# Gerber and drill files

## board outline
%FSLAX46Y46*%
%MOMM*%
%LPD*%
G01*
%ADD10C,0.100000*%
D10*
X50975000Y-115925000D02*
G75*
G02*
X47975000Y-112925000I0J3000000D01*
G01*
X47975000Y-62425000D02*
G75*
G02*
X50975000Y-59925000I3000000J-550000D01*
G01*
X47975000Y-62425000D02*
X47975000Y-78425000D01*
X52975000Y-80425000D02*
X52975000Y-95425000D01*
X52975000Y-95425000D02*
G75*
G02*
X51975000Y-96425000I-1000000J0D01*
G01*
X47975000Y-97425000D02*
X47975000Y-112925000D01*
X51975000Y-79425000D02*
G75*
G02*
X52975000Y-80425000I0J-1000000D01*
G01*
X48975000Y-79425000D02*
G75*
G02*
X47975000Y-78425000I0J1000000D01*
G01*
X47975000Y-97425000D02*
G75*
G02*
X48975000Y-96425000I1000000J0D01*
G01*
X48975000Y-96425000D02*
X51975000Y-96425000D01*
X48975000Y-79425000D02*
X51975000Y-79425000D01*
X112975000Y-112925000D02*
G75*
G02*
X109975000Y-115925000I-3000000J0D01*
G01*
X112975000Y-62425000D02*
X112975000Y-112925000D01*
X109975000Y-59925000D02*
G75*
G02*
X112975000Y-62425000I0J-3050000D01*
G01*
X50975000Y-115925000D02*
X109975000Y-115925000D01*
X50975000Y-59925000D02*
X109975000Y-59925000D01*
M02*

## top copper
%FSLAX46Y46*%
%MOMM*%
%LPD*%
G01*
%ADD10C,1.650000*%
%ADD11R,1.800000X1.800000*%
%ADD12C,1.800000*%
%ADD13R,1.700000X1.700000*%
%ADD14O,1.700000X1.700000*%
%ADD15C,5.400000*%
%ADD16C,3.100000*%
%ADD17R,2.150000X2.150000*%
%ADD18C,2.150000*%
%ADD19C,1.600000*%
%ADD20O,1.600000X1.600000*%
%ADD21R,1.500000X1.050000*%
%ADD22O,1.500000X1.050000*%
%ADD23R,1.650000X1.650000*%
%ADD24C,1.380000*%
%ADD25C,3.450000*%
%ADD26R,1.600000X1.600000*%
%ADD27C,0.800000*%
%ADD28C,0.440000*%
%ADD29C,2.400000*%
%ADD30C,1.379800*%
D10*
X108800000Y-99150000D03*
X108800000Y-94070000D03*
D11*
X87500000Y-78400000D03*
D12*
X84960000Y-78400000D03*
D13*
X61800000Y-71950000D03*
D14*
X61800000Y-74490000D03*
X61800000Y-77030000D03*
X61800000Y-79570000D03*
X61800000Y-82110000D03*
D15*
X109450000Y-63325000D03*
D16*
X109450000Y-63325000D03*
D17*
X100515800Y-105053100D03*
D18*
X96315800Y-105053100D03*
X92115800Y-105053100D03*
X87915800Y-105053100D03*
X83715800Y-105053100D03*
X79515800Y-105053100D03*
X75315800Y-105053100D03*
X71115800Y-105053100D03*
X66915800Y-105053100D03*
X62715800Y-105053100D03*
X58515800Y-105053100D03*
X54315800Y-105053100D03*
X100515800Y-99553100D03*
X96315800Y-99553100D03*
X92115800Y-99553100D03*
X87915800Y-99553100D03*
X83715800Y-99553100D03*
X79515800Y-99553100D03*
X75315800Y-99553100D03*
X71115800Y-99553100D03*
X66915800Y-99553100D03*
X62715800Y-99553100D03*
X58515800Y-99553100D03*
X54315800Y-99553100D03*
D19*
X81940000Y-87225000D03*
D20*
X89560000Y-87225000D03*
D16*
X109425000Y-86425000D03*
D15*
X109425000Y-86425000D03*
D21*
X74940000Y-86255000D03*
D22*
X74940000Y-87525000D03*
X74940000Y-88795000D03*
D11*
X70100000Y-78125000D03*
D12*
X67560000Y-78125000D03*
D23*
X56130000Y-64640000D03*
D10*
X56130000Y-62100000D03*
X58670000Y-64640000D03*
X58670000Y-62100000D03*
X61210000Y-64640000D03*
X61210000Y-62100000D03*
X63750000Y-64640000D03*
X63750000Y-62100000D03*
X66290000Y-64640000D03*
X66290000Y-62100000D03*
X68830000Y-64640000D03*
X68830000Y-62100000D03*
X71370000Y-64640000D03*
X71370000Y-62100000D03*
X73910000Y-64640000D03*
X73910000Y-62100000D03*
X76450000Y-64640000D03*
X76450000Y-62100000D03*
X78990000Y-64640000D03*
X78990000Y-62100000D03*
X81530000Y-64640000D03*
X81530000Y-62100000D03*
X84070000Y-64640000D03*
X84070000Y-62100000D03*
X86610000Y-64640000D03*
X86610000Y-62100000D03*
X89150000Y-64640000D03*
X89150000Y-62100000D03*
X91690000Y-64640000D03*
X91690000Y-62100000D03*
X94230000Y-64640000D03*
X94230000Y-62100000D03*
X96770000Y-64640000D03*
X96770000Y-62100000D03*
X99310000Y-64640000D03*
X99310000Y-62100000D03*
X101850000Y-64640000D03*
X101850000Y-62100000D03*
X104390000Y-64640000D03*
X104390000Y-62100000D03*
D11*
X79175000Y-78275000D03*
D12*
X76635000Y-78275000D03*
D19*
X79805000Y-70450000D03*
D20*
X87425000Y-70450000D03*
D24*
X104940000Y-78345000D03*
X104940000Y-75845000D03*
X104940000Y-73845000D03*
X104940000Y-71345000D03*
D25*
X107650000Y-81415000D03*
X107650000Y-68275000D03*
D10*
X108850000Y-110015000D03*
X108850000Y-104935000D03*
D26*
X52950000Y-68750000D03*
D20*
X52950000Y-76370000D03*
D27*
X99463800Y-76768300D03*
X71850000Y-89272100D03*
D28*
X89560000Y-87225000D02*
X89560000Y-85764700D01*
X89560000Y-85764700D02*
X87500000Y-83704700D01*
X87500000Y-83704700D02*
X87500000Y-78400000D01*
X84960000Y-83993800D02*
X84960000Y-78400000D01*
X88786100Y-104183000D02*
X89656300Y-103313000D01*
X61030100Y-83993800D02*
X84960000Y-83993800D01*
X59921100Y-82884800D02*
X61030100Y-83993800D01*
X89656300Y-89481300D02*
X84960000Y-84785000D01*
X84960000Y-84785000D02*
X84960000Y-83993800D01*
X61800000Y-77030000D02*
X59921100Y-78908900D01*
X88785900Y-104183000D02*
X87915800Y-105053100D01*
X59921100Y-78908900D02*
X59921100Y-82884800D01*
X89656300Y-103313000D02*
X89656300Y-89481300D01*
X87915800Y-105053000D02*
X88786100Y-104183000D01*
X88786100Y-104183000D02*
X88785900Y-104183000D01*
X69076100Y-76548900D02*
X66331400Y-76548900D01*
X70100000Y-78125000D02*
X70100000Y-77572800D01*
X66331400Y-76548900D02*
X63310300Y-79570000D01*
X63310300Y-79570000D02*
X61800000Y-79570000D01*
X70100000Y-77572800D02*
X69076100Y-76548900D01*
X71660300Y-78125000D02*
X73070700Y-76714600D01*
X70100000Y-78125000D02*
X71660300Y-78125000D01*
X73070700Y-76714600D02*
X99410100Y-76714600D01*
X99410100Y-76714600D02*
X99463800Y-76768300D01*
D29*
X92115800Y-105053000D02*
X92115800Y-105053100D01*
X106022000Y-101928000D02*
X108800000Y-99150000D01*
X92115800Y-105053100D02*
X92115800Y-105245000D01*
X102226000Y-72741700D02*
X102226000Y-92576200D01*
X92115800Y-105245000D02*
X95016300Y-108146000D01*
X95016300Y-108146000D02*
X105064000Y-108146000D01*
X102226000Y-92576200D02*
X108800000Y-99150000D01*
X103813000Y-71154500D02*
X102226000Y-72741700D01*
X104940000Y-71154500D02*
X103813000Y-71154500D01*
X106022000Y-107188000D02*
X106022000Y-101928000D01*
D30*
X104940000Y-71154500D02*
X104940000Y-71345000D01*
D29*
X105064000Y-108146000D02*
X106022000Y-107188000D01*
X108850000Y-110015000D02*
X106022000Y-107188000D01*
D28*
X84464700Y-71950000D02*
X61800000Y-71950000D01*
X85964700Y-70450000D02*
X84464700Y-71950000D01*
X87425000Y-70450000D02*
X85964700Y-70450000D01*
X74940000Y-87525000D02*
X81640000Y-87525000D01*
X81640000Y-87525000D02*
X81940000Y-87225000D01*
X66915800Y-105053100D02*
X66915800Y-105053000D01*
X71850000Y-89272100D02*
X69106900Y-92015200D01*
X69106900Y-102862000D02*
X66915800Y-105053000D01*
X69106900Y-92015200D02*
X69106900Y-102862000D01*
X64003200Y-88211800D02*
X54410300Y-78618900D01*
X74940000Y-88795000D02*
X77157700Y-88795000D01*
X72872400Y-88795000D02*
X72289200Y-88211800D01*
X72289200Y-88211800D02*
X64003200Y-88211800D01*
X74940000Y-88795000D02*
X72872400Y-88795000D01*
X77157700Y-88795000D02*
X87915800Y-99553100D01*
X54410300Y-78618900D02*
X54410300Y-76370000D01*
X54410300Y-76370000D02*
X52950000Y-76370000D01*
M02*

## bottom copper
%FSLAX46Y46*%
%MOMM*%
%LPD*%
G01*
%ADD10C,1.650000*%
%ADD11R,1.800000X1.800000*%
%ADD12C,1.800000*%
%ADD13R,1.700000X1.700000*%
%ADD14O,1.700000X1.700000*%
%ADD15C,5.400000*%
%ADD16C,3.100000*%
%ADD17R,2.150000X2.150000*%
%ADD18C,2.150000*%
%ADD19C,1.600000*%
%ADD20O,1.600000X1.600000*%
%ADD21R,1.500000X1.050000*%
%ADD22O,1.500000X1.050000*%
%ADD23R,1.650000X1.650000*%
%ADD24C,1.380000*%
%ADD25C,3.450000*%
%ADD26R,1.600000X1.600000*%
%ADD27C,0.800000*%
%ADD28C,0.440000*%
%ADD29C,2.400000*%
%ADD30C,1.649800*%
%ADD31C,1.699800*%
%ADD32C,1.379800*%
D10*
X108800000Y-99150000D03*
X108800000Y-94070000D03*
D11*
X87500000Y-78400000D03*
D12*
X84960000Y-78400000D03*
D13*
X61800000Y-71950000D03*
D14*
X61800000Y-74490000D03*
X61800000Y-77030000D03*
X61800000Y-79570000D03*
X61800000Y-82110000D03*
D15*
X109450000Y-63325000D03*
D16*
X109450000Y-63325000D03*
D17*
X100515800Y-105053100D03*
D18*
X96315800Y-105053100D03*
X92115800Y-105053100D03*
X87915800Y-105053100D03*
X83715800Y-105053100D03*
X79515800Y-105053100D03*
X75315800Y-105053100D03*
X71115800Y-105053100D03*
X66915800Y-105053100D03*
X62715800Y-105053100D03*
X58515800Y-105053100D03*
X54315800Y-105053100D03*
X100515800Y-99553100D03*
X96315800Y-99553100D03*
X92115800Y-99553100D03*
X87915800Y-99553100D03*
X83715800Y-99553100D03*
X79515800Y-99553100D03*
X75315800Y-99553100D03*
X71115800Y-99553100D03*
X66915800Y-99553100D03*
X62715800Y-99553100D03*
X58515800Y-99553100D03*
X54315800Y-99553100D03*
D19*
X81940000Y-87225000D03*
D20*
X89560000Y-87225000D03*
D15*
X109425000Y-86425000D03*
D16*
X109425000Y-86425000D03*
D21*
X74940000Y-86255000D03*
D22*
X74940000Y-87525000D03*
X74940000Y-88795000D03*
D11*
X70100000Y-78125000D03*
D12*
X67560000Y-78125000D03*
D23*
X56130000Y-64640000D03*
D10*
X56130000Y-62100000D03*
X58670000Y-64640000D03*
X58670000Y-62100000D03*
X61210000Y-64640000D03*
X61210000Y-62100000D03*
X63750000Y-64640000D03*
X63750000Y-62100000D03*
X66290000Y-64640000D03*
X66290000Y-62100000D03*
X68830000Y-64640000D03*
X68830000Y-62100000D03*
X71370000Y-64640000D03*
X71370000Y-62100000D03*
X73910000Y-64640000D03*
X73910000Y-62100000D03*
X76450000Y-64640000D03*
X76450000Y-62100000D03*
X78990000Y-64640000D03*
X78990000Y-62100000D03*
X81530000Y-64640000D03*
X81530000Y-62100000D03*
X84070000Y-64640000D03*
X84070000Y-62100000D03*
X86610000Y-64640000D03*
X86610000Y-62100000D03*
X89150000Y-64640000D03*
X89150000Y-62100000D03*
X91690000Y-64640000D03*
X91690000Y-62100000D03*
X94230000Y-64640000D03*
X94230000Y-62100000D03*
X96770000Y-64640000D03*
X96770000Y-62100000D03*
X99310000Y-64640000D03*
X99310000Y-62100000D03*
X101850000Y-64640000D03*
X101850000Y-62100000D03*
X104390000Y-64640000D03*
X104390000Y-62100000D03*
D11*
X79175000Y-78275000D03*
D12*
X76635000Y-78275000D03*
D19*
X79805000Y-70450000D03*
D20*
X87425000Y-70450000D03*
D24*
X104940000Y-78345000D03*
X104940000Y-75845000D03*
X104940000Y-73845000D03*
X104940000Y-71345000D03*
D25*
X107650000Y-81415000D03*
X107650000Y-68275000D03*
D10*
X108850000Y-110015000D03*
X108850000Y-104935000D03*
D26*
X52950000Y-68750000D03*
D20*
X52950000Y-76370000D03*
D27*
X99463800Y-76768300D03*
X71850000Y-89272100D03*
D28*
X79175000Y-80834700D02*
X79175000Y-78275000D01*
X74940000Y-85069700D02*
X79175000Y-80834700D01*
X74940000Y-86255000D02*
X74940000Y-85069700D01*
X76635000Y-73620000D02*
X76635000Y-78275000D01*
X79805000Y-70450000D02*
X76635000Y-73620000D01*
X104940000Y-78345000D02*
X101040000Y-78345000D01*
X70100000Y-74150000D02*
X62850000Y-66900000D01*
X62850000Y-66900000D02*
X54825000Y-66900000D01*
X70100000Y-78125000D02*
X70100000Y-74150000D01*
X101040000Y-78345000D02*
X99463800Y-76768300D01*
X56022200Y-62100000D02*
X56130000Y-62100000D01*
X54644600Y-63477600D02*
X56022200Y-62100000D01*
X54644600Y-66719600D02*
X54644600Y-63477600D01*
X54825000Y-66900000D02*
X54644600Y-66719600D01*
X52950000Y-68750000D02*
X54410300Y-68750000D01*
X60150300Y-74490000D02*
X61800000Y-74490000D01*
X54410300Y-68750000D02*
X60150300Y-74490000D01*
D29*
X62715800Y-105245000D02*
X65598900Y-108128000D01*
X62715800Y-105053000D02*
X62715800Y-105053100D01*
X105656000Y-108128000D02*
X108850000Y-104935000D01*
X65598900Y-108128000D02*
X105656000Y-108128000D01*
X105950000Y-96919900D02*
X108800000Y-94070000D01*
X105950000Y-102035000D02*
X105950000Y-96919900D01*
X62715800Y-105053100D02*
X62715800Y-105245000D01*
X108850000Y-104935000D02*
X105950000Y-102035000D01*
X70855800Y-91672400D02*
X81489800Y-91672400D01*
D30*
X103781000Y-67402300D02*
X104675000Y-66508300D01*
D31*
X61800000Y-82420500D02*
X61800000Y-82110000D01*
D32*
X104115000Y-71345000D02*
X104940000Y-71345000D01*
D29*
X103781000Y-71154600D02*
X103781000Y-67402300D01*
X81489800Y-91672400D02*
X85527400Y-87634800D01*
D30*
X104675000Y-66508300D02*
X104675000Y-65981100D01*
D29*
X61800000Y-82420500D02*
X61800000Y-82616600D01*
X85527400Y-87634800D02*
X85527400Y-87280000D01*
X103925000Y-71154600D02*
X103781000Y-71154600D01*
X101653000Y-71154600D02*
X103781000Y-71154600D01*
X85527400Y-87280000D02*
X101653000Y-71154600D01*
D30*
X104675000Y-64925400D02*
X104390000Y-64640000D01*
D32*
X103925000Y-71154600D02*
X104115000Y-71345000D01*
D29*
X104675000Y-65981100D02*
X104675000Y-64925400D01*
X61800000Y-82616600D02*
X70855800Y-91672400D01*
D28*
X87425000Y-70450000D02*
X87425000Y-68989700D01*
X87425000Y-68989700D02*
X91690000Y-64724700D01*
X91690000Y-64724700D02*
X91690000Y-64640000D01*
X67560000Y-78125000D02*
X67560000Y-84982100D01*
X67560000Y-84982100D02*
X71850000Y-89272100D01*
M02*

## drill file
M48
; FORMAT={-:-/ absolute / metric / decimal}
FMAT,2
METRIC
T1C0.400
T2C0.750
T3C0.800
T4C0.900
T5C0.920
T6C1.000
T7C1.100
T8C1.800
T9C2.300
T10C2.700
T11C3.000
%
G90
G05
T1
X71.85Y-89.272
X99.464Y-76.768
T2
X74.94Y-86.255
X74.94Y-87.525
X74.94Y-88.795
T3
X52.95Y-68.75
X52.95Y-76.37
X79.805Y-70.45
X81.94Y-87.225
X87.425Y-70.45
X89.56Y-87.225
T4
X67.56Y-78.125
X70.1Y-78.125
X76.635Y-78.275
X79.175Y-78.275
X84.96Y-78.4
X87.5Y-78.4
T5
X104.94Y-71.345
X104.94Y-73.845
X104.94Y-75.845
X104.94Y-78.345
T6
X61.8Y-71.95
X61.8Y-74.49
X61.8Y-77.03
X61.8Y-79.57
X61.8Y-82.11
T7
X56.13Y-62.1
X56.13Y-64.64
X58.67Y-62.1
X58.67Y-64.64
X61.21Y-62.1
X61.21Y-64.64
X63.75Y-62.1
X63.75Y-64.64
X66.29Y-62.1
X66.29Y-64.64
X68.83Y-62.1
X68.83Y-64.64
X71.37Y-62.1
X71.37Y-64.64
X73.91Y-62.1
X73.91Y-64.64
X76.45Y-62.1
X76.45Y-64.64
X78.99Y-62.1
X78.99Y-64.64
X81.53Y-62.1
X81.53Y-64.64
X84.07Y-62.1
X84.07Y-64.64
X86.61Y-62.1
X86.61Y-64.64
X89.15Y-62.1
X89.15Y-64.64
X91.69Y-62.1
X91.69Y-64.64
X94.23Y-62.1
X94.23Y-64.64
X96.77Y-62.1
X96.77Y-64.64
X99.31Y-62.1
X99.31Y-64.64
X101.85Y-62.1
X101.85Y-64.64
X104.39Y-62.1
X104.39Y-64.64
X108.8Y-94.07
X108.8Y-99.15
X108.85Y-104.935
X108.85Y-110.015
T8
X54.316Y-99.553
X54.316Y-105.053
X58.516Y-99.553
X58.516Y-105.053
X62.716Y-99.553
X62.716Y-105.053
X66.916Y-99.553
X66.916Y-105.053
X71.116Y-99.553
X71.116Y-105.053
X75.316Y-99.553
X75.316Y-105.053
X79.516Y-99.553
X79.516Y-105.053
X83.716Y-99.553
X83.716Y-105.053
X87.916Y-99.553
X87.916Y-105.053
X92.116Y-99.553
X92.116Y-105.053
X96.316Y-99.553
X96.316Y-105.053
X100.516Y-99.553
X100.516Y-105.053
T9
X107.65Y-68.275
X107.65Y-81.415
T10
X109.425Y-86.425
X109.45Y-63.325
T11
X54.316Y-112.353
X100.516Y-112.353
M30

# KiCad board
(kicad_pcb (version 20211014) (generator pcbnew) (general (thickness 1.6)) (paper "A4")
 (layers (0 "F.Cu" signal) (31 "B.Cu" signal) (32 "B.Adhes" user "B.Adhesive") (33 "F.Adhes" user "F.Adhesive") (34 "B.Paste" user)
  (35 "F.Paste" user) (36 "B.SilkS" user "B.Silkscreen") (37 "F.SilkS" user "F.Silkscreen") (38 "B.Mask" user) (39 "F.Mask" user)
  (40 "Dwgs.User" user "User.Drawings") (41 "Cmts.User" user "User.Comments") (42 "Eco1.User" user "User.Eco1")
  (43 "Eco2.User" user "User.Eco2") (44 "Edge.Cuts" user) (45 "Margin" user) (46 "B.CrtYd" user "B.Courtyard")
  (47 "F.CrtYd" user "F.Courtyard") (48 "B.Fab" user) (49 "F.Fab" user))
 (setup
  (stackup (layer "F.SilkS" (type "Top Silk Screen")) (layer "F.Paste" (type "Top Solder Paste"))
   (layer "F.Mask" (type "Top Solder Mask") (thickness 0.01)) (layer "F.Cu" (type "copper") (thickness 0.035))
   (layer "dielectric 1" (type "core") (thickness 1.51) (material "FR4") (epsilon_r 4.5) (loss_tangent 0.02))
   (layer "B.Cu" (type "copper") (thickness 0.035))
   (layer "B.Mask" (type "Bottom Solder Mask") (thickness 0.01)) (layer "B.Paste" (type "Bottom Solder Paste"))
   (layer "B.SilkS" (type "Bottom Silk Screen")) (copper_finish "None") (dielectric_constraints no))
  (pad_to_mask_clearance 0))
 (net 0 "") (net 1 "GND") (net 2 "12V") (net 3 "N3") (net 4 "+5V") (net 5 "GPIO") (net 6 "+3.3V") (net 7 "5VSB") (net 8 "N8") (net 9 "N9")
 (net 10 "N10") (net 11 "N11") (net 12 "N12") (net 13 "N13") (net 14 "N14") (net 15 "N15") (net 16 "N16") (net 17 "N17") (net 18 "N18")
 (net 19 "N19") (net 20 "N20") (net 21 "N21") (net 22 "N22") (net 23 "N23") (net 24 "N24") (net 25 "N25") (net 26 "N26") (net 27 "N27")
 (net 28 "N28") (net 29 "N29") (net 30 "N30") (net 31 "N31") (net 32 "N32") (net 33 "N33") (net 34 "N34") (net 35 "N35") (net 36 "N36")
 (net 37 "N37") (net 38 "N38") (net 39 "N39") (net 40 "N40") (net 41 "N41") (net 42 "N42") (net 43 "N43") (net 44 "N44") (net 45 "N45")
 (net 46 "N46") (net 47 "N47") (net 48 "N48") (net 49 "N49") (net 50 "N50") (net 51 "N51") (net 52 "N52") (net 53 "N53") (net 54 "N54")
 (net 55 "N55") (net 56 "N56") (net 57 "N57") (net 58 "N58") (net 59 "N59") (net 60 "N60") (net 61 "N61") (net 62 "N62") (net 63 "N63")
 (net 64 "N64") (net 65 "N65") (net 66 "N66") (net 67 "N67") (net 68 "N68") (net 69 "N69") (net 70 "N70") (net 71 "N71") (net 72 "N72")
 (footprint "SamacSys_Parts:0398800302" (layer "F.Cu") (at 108.8 99.15 90)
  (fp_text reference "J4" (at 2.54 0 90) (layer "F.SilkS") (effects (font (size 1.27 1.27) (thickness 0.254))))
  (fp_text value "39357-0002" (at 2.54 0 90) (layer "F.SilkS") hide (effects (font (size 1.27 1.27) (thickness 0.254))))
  (pad "1" thru_hole circle locked (at 0 0 90) (size 1.65 1.65) (drill 1.1) (layers *.Cu *.Mask) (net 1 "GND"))
  (pad "2" thru_hole circle locked (at 5.08 0 90) (size 1.65 1.65) (drill 1.1) (layers *.Cu *.Mask) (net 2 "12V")))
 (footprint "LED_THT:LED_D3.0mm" (layer "F.Cu") (at 87.5 78.4 180)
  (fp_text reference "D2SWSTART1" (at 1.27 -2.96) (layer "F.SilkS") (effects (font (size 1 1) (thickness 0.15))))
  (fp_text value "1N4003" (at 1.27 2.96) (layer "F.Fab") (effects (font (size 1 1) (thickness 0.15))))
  (pad "1" thru_hole rect (at 0 0 180) (size 1.8 1.8) (drill 0.9) (layers *.Cu *.Mask) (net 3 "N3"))
  (pad "2" thru_hole circle (at 2.54 0 180) (size 1.8 1.8) (drill 0.9) (layers *.Cu *.Mask) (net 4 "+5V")))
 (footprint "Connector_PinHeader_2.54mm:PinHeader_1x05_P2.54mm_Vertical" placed (layer "F.Cu") (at 61.8 71.95)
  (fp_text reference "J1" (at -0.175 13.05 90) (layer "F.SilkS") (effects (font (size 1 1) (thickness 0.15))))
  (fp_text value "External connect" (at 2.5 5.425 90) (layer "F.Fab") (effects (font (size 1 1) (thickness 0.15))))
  (pad "1" thru_hole rect (at 0 0) (size 1.7 1.7) (drill 1) (layers *.Cu *.Mask) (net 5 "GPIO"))
  (pad "2" thru_hole oval (at 0 2.54) (size 1.7 1.7) (drill 1) (layers *.Cu *.Mask) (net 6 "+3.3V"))
  (pad "3" thru_hole oval (at 0 5.08) (size 1.7 1.7) (drill 1) (layers *.Cu *.Mask) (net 4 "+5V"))
  (pad "4" thru_hole oval (at 0 7.62) (size 1.7 1.7) (drill 1) (layers *.Cu *.Mask) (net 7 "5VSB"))
  (pad "5" thru_hole oval (at 0 10.16) (size 1.7 1.7) (drill 1) (layers *.Cu *.Mask) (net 1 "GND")))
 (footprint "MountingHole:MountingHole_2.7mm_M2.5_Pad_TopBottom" (layer "F.Cu") (at 109.45 63.325)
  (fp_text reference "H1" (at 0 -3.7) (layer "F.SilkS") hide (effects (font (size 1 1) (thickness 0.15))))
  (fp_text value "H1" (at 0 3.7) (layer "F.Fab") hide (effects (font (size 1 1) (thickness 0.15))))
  (pad "1" connect circle (at 0 0) (size 5.4 5.4) (layers "B.Cu" "B.Mask"))
  (pad "1" connect circle (at 0 0) (size 5.4 5.4) (layers "F.Cu" "F.Mask"))
  (pad "1" thru_hole circle (at 0 0) (size 3.1 3.1) (drill 2.7) (layers *.Cu *.Mask)))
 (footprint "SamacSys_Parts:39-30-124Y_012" (layer "F.Cu") (at 100.5158 105.0531)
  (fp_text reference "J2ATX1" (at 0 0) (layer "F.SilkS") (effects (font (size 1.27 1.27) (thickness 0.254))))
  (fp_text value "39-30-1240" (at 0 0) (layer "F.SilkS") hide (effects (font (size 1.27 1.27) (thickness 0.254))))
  (pad "" np_thru_hole circle locked (at 0 7.3) (size 3 3) (drill 3) (layers *.Cu *.Mask))
  (pad "" np_thru_hole circle locked (at -46.2 7.3) (size 3 3) (drill 3) (layers *.Cu *.Mask))
  (pad "1" thru_hole rect locked (at 0 0) (size 2.15 2.15) (drill 1.8) (layers *.Cu *.Mask) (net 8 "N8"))
  (pad "2" thru_hole circle locked (at -4.2 0) (size 2.15 2.15) (drill 1.8) (layers *.Cu *.Mask) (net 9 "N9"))
  (pad "3" thru_hole circle locked (at -8.4 0) (size 2.15 2.15) (drill 1.8) (layers *.Cu *.Mask) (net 1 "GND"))
  (pad "4" thru_hole circle locked (at -12.6 0) (size 2.15 2.15) (drill 1.8) (layers *.Cu *.Mask) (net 4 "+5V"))
  (pad "5" thru_hole circle locked (at -16.8 0) (size 2.15 2.15) (drill 1.8) (layers *.Cu *.Mask) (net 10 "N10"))
  (pad "6" thru_hole circle locked (at -21 0) (size 2.15 2.15) (drill 1.8) (layers *.Cu *.Mask) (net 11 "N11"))
  (pad "7" thru_hole circle locked (at -25.2 0) (size 2.15 2.15) (drill 1.8) (layers *.Cu *.Mask) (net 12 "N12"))
  (pad "8" thru_hole circle locked (at -29.4 0) (size 2.15 2.15) (drill 1.8) (layers *.Cu *.Mask) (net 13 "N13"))
  (pad "9" thru_hole circle locked (at -33.6 0) (size 2.15 2.15) (drill 1.8) (layers *.Cu *.Mask) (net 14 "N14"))
  (pad "10" thru_hole circle locked (at -37.8 0) (size 2.15 2.15) (drill 1.8) (layers *.Cu *.Mask) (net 2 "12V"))
  (pad "11" thru_hole circle locked (at -42 0) (size 2.15 2.15) (drill 1.8) (layers *.Cu *.Mask) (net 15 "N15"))
  (pad "12" thru_hole circle locked (at -46.2 0) (size 2.15 2.15) (drill 1.8) (layers *.Cu *.Mask) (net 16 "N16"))
  (pad "13" thru_hole circle locked (at 0 -5.5) (size 2.15 2.15) (drill 1.8) (layers *.Cu *.Mask) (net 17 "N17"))
  (pad "14" thru_hole circle locked (at -4.2 -5.5) (size 2.15 2.15) (drill 1.8) (layers *.Cu *.Mask) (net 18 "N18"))
  (pad "15" thru_hole circle locked (at -8.4 -5.5) (size 2.15 2.15) (drill 1.8) (layers *.Cu *.Mask) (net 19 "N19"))
  (pad "16" thru_hole circle locked (at -12.6 -5.5) (size 2.15 2.15) (drill 1.8) (layers *.Cu *.Mask) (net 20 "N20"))
  (pad "17" thru_hole circle locked (at -16.8 -5.5) (size 2.15 2.15) (drill 1.8) (layers *.Cu *.Mask) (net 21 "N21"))
  (pad "18" thru_hole circle locked (at -21 -5.5) (size 2.15 2.15) (drill 1.8) (layers *.Cu *.Mask) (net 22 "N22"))
  (pad "19" thru_hole circle locked (at -25.2 -5.5) (size 2.15 2.15) (drill 1.8) (layers *.Cu *.Mask) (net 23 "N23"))
  (pad "20" thru_hole circle locked (at -29.4 -5.5) (size 2.15 2.15) (drill 1.8) (layers *.Cu *.Mask) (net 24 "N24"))
  (pad "21" thru_hole circle locked (at -33.6 -5.5) (size 2.15 2.15) (drill 1.8) (layers *.Cu *.Mask) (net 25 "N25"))
  (pad "22" thru_hole circle locked (at -37.8 -5.5) (size 2.15 2.15) (drill 1.8) (layers *.Cu *.Mask) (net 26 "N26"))
  (pad "23" thru_hole circle locked (at -42 -5.5) (size 2.15 2.15) (drill 1.8) (layers *.Cu *.Mask) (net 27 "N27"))
  (pad "24" thru_hole circle locked (at -46.2 -5.5) (size 2.15 2.15) (drill 1.8) (layers *.Cu *.Mask) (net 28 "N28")))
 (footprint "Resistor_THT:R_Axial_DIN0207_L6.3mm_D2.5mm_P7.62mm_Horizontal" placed (layer "F.Cu") (at 81.94 87.225)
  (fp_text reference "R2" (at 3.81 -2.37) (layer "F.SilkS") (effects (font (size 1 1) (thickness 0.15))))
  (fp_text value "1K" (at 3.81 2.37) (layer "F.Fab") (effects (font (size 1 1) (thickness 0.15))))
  (pad "1" thru_hole circle (at 0 0) (size 1.6 1.6) (drill 0.8) (layers *.Cu *.Mask) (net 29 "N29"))
  (pad "2" thru_hole oval (at 7.62 0) (size 1.6 1.6) (drill 0.8) (layers *.Cu *.Mask) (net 3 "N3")))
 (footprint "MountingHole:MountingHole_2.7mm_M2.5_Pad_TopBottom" (layer "F.Cu") (at 109.425 86.425)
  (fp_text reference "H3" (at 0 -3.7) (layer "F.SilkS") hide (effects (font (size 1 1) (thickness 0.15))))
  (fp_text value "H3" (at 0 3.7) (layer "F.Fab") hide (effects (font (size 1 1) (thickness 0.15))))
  (pad "1" connect circle (at 0 0) (size 5.4 5.4) (layers "B.Cu" "B.Mask"))
  (pad "3" thru_hole circle (at 0 0) (size 3.1 3.1) (drill 2.7) (layers *.Cu *.Mask))
  (pad "3" connect circle (at 0 0) (size 5.4 5.4) (layers "F.Cu" "F.Mask")))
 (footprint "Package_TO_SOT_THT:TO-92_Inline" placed (layer "F.Cu") (at 74.94 86.255 -90)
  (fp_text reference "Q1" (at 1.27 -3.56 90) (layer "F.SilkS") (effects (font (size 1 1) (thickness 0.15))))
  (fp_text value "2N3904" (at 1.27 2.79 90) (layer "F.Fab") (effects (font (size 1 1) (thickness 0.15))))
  (pad "1" thru_hole rect (at 0 0 270) (size 1.05 1.5) (drill 0.75) (layers *.Cu *.Mask) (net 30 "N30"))
  (pad "2" thru_hole oval (at 1.27 0 270) (size 1.05 1.5) (drill 0.75) (layers *.Cu *.Mask) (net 29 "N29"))
  (pad "3" thru_hole oval (at 2.54 0 270) (size 1.05 1.5) (drill 0.75) (layers *.Cu *.Mask) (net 20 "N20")))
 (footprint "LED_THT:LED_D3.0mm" (layer "F.Cu") (at 70.1 78.125 180)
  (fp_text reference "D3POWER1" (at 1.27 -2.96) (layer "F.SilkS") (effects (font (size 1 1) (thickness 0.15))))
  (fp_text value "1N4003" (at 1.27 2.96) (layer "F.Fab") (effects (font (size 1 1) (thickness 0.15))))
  (pad "1" thru_hole rect (at 0 0 180) (size 1.8 1.8) (drill 0.9) (layers *.Cu *.Mask) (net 7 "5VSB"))
  (pad "2" thru_hole circle (at 2.54 0 180) (size 1.8 1.8) (drill 0.9) (layers *.Cu *.Mask) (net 14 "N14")))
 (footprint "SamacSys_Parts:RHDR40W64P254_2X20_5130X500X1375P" (layer "F.Cu") (at 56.13 64.64)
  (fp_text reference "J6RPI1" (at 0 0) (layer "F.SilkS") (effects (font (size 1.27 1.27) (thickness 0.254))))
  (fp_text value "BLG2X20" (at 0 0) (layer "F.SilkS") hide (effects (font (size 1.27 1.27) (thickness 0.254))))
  (pad "1" thru_hole rect locked (at 0 0) (size 1.65 1.65) (drill 1.1) (layers *.Cu *.Mask) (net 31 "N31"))
  (pad "2" thru_hole circle locked (at 0 -2.54) (size 1.65 1.65) (drill 1.1) (layers *.Cu *.Mask) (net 7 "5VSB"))
  (pad "3" thru_hole circle locked (at 2.54 0) (size 1.65 1.65) (drill 1.1) (layers *.Cu *.Mask) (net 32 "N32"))
  (pad "4" thru_hole circle locked (at 2.54 -2.54) (size 1.65 1.65) (drill 1.1) (layers *.Cu *.Mask) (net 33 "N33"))
  (pad "5" thru_hole circle locked (at 5.08 0) (size 1.65 1.65) (drill 1.1) (layers *.Cu *.Mask) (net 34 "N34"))
  (pad "6" thru_hole circle locked (at 5.08 -2.54) (size 1.65 1.65) (drill 1.1) (layers *.Cu *.Mask) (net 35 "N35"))
  (pad "7" thru_hole circle locked (at 7.62 0) (size 1.65 1.65) (drill 1.1) (layers *.Cu *.Mask) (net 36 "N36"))
  (pad "8" thru_hole circle locked (at 7.62 -2.54) (size 1.65 1.65) (drill 1.1) (layers *.Cu *.Mask) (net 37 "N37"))
  (pad "9" thru_hole circle locked (at 10.16 0) (size 1.65 1.65) (drill 1.1) (layers *.Cu *.Mask) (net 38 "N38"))
  (pad "10" thru_hole circle locked (at 10.16 -2.54) (size 1.65 1.65) (drill 1.1) (layers *.Cu *.Mask) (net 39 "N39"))
  (pad "11" thru_hole circle locked (at 12.7 0) (size 1.65 1.65) (drill 1.1) (layers *.Cu *.Mask) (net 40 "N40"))
  (pad "12" thru_hole circle locked (at 12.7 -2.54) (size 1.65 1.65) (drill 1.1) (layers *.Cu *.Mask) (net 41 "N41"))
  (pad "13" thru_hole circle locked (at 15.24 0) (size 1.65 1.65) (drill 1.1) (layers *.Cu *.Mask) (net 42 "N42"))
  (pad "14" thru_hole circle locked (at 15.24 -2.54) (size 1.65 1.65) (drill 1.1) (layers *.Cu *.Mask) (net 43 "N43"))
  (pad "15" thru_hole circle locked (at 17.78 0) (size 1.65 1.65) (drill 1.1) (layers *.Cu *.Mask) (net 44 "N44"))
  (pad "16" thru_hole circle locked (at 17.78 -2.54) (size 1.65 1.65) (drill 1.1) (layers *.Cu *.Mask) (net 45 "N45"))
  (pad "17" thru_hole circle locked (at 20.32 0) (size 1.65 1.65) (drill 1.1) (layers *.Cu *.Mask) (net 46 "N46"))
  (pad "18" thru_hole circle locked (at 20.32 -2.54) (size 1.65 1.65) (drill 1.1) (layers *.Cu *.Mask) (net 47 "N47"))
  (pad "19" thru_hole circle locked (at 22.86 0) (size 1.65 1.65) (drill 1.1) (layers *.Cu *.Mask) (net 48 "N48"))
  (pad "20" thru_hole circle locked (at 22.86 -2.54) (size 1.65 1.65) (drill 1.1) (layers *.Cu *.Mask) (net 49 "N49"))
  (pad "21" thru_hole circle locked (at 25.4 0) (size 1.65 1.65) (drill 1.1) (layers *.Cu *.Mask) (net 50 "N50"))
  (pad "22" thru_hole circle locked (at 25.4 -2.54) (size 1.65 1.65) (drill 1.1) (layers *.Cu *.Mask) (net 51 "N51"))
  (pad "23" thru_hole circle locked (at 27.94 0) (size 1.65 1.65) (drill 1.1) (layers *.Cu *.Mask) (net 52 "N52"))
  (pad "24" thru_hole circle locked (at 27.94 -2.54) (size 1.65 1.65) (drill 1.1) (layers *.Cu *.Mask) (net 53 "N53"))
  (pad "25" thru_hole circle locked (at 30.48 0) (size 1.65 1.65) (drill 1.1) (layers *.Cu *.Mask) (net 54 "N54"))
  (pad "26" thru_hole circle locked (at 30.48 -2.54) (size 1.65 1.65) (drill 1.1) (layers *.Cu *.Mask) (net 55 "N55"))
  (pad "27" thru_hole circle locked (at 33.02 0) (size 1.65 1.65) (drill 1.1) (layers *.Cu *.Mask) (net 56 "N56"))
  (pad "28" thru_hole circle locked (at 33.02 -2.54) (size 1.65 1.65) (drill 1.1) (layers *.Cu *.Mask) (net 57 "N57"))
  (pad "29" thru_hole circle locked (at 35.56 0) (size 1.65 1.65) (drill 1.1) (layers *.Cu *.Mask) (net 5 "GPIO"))
  (pad "30" thru_hole circle locked (at 35.56 -2.54) (size 1.65 1.65) (drill 1.1) (layers *.Cu *.Mask) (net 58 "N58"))
  (pad "31" thru_hole circle locked (at 38.1 0) (size 1.65 1.65) (drill 1.1) (layers *.Cu *.Mask) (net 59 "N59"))
  (pad "32" thru_hole circle locked (at 38.1 -2.54) (size 1.65 1.65) (drill 1.1) (layers *.Cu *.Mask) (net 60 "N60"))
  (pad "33" thru_hole circle locked (at 40.64 0) (size 1.65 1.65) (drill 1.1) (layers *.Cu *.Mask) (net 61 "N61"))
  (pad "34" thru_hole circle locked (at 40.64 -2.54) (size 1.65 1.65) (drill 1.1) (layers *.Cu *.Mask) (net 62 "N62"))
  (pad "35" thru_hole circle locked (at 43.18 0) (size 1.65 1.65) (drill 1.1) (layers *.Cu *.Mask) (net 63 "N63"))
  (pad "36" thru_hole circle locked (at 43.18 -2.54) (size 1.65 1.65) (drill 1.1) (layers *.Cu *.Mask) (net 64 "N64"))
  (pad "37" thru_hole circle locked (at 45.72 0) (size 1.65 1.65) (drill 1.1) (layers *.Cu *.Mask) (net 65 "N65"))
  (pad "38" thru_hole circle locked (at 45.72 -2.54) (size 1.65 1.65) (drill 1.1) (layers *.Cu *.Mask) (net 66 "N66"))
  (pad "39" thru_hole circle locked (at 48.26 0) (size 1.65 1.65) (drill 1.1) (layers *.Cu *.Mask) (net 1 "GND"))
  (pad "40" thru_hole circle locked (at 48.26 -2.54) (size 1.65 1.65) (drill 1.1) (layers *.Cu *.Mask) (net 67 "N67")))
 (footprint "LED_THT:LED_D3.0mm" (layer "F.Cu") (at 79.175 78.275 180)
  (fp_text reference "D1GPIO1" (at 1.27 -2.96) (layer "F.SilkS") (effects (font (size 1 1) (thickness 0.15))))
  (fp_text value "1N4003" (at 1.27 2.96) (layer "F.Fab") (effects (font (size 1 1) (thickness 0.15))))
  (pad "1" thru_hole rect (at 0 0 180) (size 1.8 1.8) (drill 0.9) (layers *.Cu *.Mask) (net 30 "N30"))
  (pad "2" thru_hole circle (at 2.54 0 180) (size 1.8 1.8) (drill 0.9) (layers *.Cu *.Mask) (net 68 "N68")))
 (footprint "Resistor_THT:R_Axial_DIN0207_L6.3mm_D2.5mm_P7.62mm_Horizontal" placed (layer "F.Cu") (at 79.805 70.45)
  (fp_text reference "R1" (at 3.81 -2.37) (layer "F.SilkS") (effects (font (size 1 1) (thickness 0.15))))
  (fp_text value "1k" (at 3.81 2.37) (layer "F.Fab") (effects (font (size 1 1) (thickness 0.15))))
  (pad "1" thru_hole circle (at 0 0) (size 1.6 1.6) (drill 0.8) (layers *.Cu *.Mask) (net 68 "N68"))
  (pad "2" thru_hole oval (at 7.62 0) (size 1.6 1.6) (drill 0.8) (layers *.Cu *.Mask) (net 5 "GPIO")))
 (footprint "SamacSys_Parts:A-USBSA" (layer "F.Cu") (at 110.95 74.845 90)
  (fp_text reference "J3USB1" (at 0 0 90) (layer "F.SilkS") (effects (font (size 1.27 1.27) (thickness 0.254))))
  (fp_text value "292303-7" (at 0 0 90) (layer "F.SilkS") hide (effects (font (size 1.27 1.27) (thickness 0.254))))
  (pad "1" thru_hole circle locked (at -3.5 -6.01 90) (size 1.38 1.38) (drill 0.92) (layers *.Cu *.Mask) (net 7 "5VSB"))
  (pad "2" thru_hole circle locked (at -1 -6.01 90) (size 1.38 1.38) (drill 0.92) (layers *.Cu *.Mask) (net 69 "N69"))
  (pad "3" thru_hole circle locked (at 1 -6.01 90) (size 1.38 1.38) (drill 0.92) (layers *.Cu *.Mask) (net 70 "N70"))
  (pad "4" thru_hole circle locked (at 3.5 -6.01 90) (size 1.38 1.38) (drill 0.92) (layers *.Cu *.Mask) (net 1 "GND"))
  (pad "5" thru_hole circle locked (at -6.57 -3.3 90) (size 3.45 3.45) (drill 2.3) (layers *.Cu *.Mask) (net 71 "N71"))
  (pad "6" thru_hole circle locked (at 6.57 -3.3 90) (size 3.45 3.45) (drill 2.3) (layers *.Cu *.Mask) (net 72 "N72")))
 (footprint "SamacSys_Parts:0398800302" (layer "F.Cu") (at 108.85 110.015 90)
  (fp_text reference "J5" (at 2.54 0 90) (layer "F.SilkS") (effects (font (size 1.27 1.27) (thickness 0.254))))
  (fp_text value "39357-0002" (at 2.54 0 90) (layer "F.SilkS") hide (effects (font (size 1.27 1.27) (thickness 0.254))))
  (pad "1" thru_hole circle locked (at 0 0 90) (size 1.65 1.65) (drill 1.1) (layers *.Cu *.Mask) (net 1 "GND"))
  (pad "2" thru_hole circle locked (at 5.08 0 90) (size 1.65 1.65) (drill 1.1) (layers *.Cu *.Mask) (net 2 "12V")))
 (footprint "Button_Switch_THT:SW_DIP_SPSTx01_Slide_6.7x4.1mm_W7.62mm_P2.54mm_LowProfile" (layer "F.Cu") (at 52.95 68.75 -90)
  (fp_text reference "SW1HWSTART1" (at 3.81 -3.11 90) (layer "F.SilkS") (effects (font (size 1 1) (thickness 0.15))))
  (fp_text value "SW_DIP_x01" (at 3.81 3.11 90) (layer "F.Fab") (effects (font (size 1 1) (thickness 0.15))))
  (pad "1" thru_hole rect (at 0 0 270) (size 1.6 1.6) (drill 0.8) (layers *.Cu *.Mask) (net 6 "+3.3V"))
  (pad "2" thru_hole oval (at 7.62 0 270) (size 1.6 1.6) (drill 0.8) (layers *.Cu *.Mask) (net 20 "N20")))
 (gr_arc (start 50.975 115.925) (mid 48.85368 115.04632) (end 47.975 112.925) (layer "Edge.Cuts") (width 0.1))
 (gr_arc (start 47.975 62.425) (mid 49.022438 60.631925) (end 50.975 59.925) (layer "Edge.Cuts") (width 0.1))
 (gr_line (start 47.975 62.425) (end 47.975 78.425) (layer "Edge.Cuts") (width 0.1))
 (gr_line (start 52.975 80.425) (end 52.975 95.425) (layer "Edge.Cuts") (width 0.1))
 (gr_arc (start 52.975 95.425) (mid 52.682107 96.132107) (end 51.975 96.425) (layer "Edge.Cuts") (width 0.1))
 (gr_line (start 47.975 97.425) (end 47.975 112.925) (layer "Edge.Cuts") (width 0.1))
 (gr_arc (start 51.975 79.425) (mid 52.682107 79.717893) (end 52.975 80.425) (layer "Edge.Cuts") (width 0.1))
 (gr_arc (start 48.975 79.425) (mid 48.267893 79.132107) (end 47.975 78.425) (layer "Edge.Cuts") (width 0.1))
 (gr_arc (start 47.975 97.425) (mid 48.267893 96.717893) (end 48.975 96.425) (layer "Edge.Cuts") (width 0.1))
 (gr_line (start 48.975 96.425) (end 51.975 96.425) (layer "Edge.Cuts") (width 0.1))
 (gr_line (start 48.975 79.425) (end 51.975 79.425) (layer "Edge.Cuts") (width 0.1))
 (gr_arc (start 112.975 112.925) (mid 112.09632 115.04632) (end 109.975 115.925) (layer "Edge.Cuts") (width 0.1))
 (gr_line (start 112.975 62.425) (end 112.975 112.925) (layer "Edge.Cuts") (width 0.1))
 (gr_arc (start 109.975 59.925) (mid 111.927562 60.631925) (end 112.975 62.425) (layer "Edge.Cuts") (width 0.1))
 (gr_line (start 50.975 115.925) (end 109.975 115.925) (layer "Edge.Cuts") (width 0.1))
 (gr_line (start 50.975 59.925) (end 109.975 59.925) (layer "Edge.Cuts") (width 0.1))
 (segment (start 79.175 80.8347) (end 79.175 78.275) (width 0.44) (layer "B.Cu") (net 30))
 (segment (start 74.94 85.0697) (end 79.175 80.8347) (width 0.44) (layer "B.Cu") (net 30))
 (segment (start 74.94 86.255) (end 74.94 85.0697) (width 0.44) (layer "B.Cu") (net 30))
 (segment (start 76.635 73.62) (end 76.635 78.275) (width 0.44) (layer "B.Cu") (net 68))
 (segment (start 79.805 70.45) (end 76.635 73.62) (width 0.44) (layer "B.Cu") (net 68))
 (segment (start 89.56 87.225) (end 89.56 85.7647) (width 0.44) (layer "F.Cu") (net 3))
 (segment (start 89.56 85.7647) (end 87.5 83.7047) (width 0.44) (layer "F.Cu") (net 3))
 (segment (start 87.5 83.7047) (end 87.5 78.4) (width 0.44) (layer "F.Cu") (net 3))
 (segment (start 84.96 83.9938) (end 84.96 78.4) (width 0.44) (layer "F.Cu") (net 4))
 (segment (start 88.7861 104.183) (end 89.6563 103.313) (width 0.44) (layer "F.Cu") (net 4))
 (segment (start 61.0301 83.9938) (end 84.96 83.9938) (width 0.44) (layer "F.Cu") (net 4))
 (segment (start 59.9211 82.8848) (end 61.0301 83.9938) (width 0.44) (layer "F.Cu") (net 4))
 (segment (start 89.6563 89.4813) (end 84.96 84.785) (width 0.44) (layer "F.Cu") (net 4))
 (segment (start 84.96 84.785) (end 84.96 83.9938) (width 0.44) (layer "F.Cu") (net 4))
 (segment (start 61.8 77.03) (end 59.9211 78.9089) (width 0.44) (layer "F.Cu") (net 4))
 (segment (start 88.7859 104.183) (end 87.9158 105.0531) (width 0.44) (layer "F.Cu") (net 4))
 (segment (start 59.9211 78.9089) (end 59.9211 82.8848) (width 0.44) (layer "F.Cu") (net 4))
 (segment (start 89.6563 103.313) (end 89.6563 89.4813) (width 0.44) (layer "F.Cu") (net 4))
 (segment (start 87.9158 105.053) (end 88.7861 104.183) (width 0.44) (layer "F.Cu") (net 4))
 (segment (start 88.7861 104.183) (end 88.7859 104.183) (width 0.44) (layer "F.Cu") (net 4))
 (segment (start 69.0761 76.5489) (end 66.3314 76.5489) (width 0.44) (layer "F.Cu") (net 7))
 (segment (start 70.1 78.125) (end 70.1 77.5728) (width 0.44) (layer "F.Cu") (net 7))
 (segment (start 66.3314 76.5489) (end 63.3103 79.57) (width 0.44) (layer "F.Cu") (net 7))
 (segment (start 63.3103 79.57) (end 61.8 79.57) (width 0.44) (layer "F.Cu") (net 7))
 (segment (start 70.1 77.5728) (end 69.0761 76.5489) (width 0.44) (layer "F.Cu") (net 7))
 (segment (start 71.6603 78.125) (end 73.0707 76.7146) (width 0.44) (layer "F.Cu") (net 7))
 (segment (start 70.1 78.125) (end 71.6603 78.125) (width 0.44) (layer "F.Cu") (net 7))
 (segment (start 73.0707 76.7146) (end 99.4101 76.7146) (width 0.44) (layer "F.Cu") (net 7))
 (segment (start 99.4101 76.7146) (end 99.4638 76.7683) (width 0.44) (layer "F.Cu") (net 7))
 (via (at 99.4638 76.7683) (size 0.8) (drill 0.4) (layers "F.Cu" "B.Cu") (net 7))
 (segment (start 104.94 78.345) (end 101.04 78.345) (width 0.44) (layer "B.Cu") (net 7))
 (segment (start 70.1 74.15) (end 62.85 66.9) (width 0.44) (layer "B.Cu") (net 7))
 (segment (start 62.85 66.9) (end 54.825 66.9) (width 0.44) (layer "B.Cu") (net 7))
 (segment (start 70.1 78.125) (end 70.1 74.15) (width 0.44) (layer "B.Cu") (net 7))
 (segment (start 101.04 78.345) (end 99.4638 76.7683) (width 0.44) (layer "B.Cu") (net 7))
 (segment (start 56.0222 62.1) (end 56.13 62.1) (width 0.44) (layer "B.Cu") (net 7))
 (segment (start 54.6446 63.4776) (end 56.0222 62.1) (width 0.44) (layer "B.Cu") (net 7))
 (segment (start 54.6446 66.7196) (end 54.6446 63.4776) (width 0.44) (layer "B.Cu") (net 7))
 (segment (start 54.825 66.9) (end 54.6446 66.7196) (width 0.44) (layer "B.Cu") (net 7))
 (segment (start 52.95 68.75) (end 54.4103 68.75) (width 0.44) (layer "B.Cu") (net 6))
 (segment (start 60.1503 74.49) (end 61.8 74.49) (width 0.44) (layer "B.Cu") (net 6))
 (segment (start 54.4103 68.75) (end 60.1503 74.49) (width 0.44) (layer "B.Cu") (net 6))
 (segment (start 62.7158 105.245) (end 65.5989 108.128) (width 2.4) (layer "B.Cu") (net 2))
 (segment (start 62.7158 105.053) (end 62.7158 105.0531) (width 2.4) (layer "B.Cu") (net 2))
 (segment (start 105.656 108.128) (end 108.85 104.935) (width 2.4) (layer "B.Cu") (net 2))
 (segment (start 65.5989 108.128) (end 105.656 108.128) (width 2.4) (layer "B.Cu") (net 2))
 (segment (start 105.95 96.9199) (end 108.8 94.07) (width 2.4) (layer "B.Cu") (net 2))
 (segment (start 105.95 102.035) (end 105.95 96.9199) (width 2.4) (layer "B.Cu") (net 2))
 (segment (start 62.7158 105.0531) (end 62.7158 105.245) (width 2.4) (layer "B.Cu") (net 2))
 (segment (start 108.85 104.935) (end 105.95 102.035) (width 2.4) (layer "B.Cu") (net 2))
 (segment (start 92.1158 105.053) (end 92.1158 105.0531) (width 2.4) (layer "F.Cu") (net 1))
 (segment (start 106.022 101.928) (end 108.8 99.15) (width 2.4) (layer "F.Cu") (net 1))
 (segment (start 92.1158 105.0531) (end 92.1158 105.245) (width 2.4) (layer "F.Cu") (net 1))
 (segment (start 102.226 72.7417) (end 102.226 92.5762) (width 2.4) (layer "F.Cu") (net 1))
 (segment (start 92.1158 105.245) (end 95.0163 108.146) (width 2.4) (layer "F.Cu") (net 1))
 (segment (start 95.0163 108.146) (end 105.064 108.146) (width 2.4) (layer "F.Cu") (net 1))
 (segment (start 102.226 92.5762) (end 108.8 99.15) (width 2.4) (layer "F.Cu") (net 1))
 (segment (start 103.813 71.1545) (end 102.226 72.7417) (width 2.4) (layer "F.Cu") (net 1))
 (segment (start 104.94 71.1545) (end 103.813 71.1545) (width 2.4) (layer "F.Cu") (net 1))
 (segment (start 106.022 107.188) (end 106.022 101.928) (width 2.4) (layer "F.Cu") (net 1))
 (segment (start 104.94 71.1545) (end 104.94 71.345) (width 1.3798) (layer "F.Cu") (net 1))
 (segment (start 105.064 108.146) (end 106.022 107.188) (width 2.4) (layer "F.Cu") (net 1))
 (segment (start 108.85 110.015) (end 106.022 107.188) (width 2.4) (layer "F.Cu") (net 1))
 (segment (start 70.8558 91.6724) (end 81.4898 91.6724) (width 2.4) (layer "B.Cu") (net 1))
 (segment (start 103.781 67.4023) (end 104.675 66.5083) (width 1.6498) (layer "B.Cu") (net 1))
 (segment (start 61.8 82.4205) (end 61.8 82.11) (width 1.6998) (layer "B.Cu") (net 1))
 (segment (start 104.115 71.345) (end 104.94 71.345) (width 1.3798) (layer "B.Cu") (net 1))
 (segment (start 103.781 71.1546) (end 103.781 67.4023) (width 2.4) (layer "B.Cu") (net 1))
 (segment (start 81.4898 91.6724) (end 85.5274 87.6348) (width 2.4) (layer "B.Cu") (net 1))
 (segment (start 104.675 66.5083) (end 104.675 65.9811) (width 1.6498) (layer "B.Cu") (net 1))
 (segment (start 61.8 82.4205) (end 61.8 82.6166) (width 2.4) (layer "B.Cu") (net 1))
 (segment (start 85.5274 87.6348) (end 85.5274 87.28) (width 2.4) (layer "B.Cu") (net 1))
 (segment (start 103.925 71.1546) (end 103.781 71.1546) (width 2.4) (layer "B.Cu") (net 1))
 (segment (start 101.653 71.1546) (end 103.781 71.1546) (width 2.4) (layer "B.Cu") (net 1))
 (segment (start 85.5274 87.28) (end 101.653 71.1546) (width 2.4) (layer "B.Cu") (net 1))
 (segment (start 104.675 64.9254) (end 104.39 64.64) (width 1.6498) (layer "B.Cu") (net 1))
 (segment (start 103.925 71.1546) (end 104.115 71.345) (width 1.3798) (layer "B.Cu") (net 1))
 (segment (start 104.675 65.9811) (end 104.675 64.9254) (width 2.4) (layer "B.Cu") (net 1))
 (segment (start 61.8 82.6166) (end 70.8558 91.6724) (width 2.4) (layer "B.Cu") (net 1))
 (segment (start 84.4647 71.95) (end 61.8 71.95) (width 0.44) (layer "F.Cu") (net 5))
 (segment (start 85.9647 70.45) (end 84.4647 71.95) (width 0.44) (layer "F.Cu") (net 5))
 (segment (start 87.425 70.45) (end 85.9647 70.45) (width 0.44) (layer "F.Cu") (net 5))
 (segment (start 87.425 70.45) (end 87.425 68.9897) (width 0.44) (layer "B.Cu") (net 5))
 (segment (start 87.425 68.9897) (end 91.69 64.7247) (width 0.44) (layer "B.Cu") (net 5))
 (segment (start 91.69 64.7247) (end 91.69 64.64) (width 0.44) (layer "B.Cu") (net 5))
 (segment (start 74.94 87.525) (end 81.64 87.525) (width 0.44) (layer "F.Cu") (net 29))
 (segment (start 81.64 87.525) (end 81.94 87.225) (width 0.44) (layer "F.Cu") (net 29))
 (segment (start 66.9158 105.0531) (end 66.9158 105.053) (width 0.44) (layer "F.Cu") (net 14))
 (segment (start 71.85 89.2721) (end 69.1069 92.0152) (width 0.44) (layer "F.Cu") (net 14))
 (segment (start 69.1069 102.862) (end 66.9158 105.053) (width 0.44) (layer "F.Cu") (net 14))
 (segment (start 69.1069 92.0152) (end 69.1069 102.862) (width 0.44) (layer "F.Cu") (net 14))
 (via (at 71.85 89.2721) (size 0.8) (drill 0.4) (layers "F.Cu" "B.Cu") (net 14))
 (segment (start 67.56 78.125) (end 67.56 84.9821) (width 0.44) (layer "B.Cu") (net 14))
 (segment (start 67.56 84.9821) (end 71.85 89.2721) (width 0.44) (layer "B.Cu") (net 14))
 (segment (start 64.0032 88.2118) (end 54.4103 78.6189) (width 0.44) (layer "F.Cu") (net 20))
 (segment (start 74.94 88.795) (end 77.1577 88.795) (width 0.44) (layer "F.Cu") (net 20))
 (segment (start 72.8724 88.795) (end 72.2892 88.2118) (width 0.44) (layer "F.Cu") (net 20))
 (segment (start 72.2892 88.2118) (end 64.0032 88.2118) (width 0.44) (layer "F.Cu") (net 20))
 (segment (start 74.94 88.795) (end 72.8724 88.795) (width 0.44) (layer "F.Cu") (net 20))
 (segment (start 77.1577 88.795) (end 87.9158 99.5531) (width 0.44) (layer "F.Cu") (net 20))
 (segment (start 54.4103 78.6189) (end 54.4103 76.37) (width 0.44) (layer "F.Cu") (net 20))
 (segment (start 54.4103 76.37) (end 52.95 76.37) (width 0.44) (layer "F.Cu") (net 20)))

